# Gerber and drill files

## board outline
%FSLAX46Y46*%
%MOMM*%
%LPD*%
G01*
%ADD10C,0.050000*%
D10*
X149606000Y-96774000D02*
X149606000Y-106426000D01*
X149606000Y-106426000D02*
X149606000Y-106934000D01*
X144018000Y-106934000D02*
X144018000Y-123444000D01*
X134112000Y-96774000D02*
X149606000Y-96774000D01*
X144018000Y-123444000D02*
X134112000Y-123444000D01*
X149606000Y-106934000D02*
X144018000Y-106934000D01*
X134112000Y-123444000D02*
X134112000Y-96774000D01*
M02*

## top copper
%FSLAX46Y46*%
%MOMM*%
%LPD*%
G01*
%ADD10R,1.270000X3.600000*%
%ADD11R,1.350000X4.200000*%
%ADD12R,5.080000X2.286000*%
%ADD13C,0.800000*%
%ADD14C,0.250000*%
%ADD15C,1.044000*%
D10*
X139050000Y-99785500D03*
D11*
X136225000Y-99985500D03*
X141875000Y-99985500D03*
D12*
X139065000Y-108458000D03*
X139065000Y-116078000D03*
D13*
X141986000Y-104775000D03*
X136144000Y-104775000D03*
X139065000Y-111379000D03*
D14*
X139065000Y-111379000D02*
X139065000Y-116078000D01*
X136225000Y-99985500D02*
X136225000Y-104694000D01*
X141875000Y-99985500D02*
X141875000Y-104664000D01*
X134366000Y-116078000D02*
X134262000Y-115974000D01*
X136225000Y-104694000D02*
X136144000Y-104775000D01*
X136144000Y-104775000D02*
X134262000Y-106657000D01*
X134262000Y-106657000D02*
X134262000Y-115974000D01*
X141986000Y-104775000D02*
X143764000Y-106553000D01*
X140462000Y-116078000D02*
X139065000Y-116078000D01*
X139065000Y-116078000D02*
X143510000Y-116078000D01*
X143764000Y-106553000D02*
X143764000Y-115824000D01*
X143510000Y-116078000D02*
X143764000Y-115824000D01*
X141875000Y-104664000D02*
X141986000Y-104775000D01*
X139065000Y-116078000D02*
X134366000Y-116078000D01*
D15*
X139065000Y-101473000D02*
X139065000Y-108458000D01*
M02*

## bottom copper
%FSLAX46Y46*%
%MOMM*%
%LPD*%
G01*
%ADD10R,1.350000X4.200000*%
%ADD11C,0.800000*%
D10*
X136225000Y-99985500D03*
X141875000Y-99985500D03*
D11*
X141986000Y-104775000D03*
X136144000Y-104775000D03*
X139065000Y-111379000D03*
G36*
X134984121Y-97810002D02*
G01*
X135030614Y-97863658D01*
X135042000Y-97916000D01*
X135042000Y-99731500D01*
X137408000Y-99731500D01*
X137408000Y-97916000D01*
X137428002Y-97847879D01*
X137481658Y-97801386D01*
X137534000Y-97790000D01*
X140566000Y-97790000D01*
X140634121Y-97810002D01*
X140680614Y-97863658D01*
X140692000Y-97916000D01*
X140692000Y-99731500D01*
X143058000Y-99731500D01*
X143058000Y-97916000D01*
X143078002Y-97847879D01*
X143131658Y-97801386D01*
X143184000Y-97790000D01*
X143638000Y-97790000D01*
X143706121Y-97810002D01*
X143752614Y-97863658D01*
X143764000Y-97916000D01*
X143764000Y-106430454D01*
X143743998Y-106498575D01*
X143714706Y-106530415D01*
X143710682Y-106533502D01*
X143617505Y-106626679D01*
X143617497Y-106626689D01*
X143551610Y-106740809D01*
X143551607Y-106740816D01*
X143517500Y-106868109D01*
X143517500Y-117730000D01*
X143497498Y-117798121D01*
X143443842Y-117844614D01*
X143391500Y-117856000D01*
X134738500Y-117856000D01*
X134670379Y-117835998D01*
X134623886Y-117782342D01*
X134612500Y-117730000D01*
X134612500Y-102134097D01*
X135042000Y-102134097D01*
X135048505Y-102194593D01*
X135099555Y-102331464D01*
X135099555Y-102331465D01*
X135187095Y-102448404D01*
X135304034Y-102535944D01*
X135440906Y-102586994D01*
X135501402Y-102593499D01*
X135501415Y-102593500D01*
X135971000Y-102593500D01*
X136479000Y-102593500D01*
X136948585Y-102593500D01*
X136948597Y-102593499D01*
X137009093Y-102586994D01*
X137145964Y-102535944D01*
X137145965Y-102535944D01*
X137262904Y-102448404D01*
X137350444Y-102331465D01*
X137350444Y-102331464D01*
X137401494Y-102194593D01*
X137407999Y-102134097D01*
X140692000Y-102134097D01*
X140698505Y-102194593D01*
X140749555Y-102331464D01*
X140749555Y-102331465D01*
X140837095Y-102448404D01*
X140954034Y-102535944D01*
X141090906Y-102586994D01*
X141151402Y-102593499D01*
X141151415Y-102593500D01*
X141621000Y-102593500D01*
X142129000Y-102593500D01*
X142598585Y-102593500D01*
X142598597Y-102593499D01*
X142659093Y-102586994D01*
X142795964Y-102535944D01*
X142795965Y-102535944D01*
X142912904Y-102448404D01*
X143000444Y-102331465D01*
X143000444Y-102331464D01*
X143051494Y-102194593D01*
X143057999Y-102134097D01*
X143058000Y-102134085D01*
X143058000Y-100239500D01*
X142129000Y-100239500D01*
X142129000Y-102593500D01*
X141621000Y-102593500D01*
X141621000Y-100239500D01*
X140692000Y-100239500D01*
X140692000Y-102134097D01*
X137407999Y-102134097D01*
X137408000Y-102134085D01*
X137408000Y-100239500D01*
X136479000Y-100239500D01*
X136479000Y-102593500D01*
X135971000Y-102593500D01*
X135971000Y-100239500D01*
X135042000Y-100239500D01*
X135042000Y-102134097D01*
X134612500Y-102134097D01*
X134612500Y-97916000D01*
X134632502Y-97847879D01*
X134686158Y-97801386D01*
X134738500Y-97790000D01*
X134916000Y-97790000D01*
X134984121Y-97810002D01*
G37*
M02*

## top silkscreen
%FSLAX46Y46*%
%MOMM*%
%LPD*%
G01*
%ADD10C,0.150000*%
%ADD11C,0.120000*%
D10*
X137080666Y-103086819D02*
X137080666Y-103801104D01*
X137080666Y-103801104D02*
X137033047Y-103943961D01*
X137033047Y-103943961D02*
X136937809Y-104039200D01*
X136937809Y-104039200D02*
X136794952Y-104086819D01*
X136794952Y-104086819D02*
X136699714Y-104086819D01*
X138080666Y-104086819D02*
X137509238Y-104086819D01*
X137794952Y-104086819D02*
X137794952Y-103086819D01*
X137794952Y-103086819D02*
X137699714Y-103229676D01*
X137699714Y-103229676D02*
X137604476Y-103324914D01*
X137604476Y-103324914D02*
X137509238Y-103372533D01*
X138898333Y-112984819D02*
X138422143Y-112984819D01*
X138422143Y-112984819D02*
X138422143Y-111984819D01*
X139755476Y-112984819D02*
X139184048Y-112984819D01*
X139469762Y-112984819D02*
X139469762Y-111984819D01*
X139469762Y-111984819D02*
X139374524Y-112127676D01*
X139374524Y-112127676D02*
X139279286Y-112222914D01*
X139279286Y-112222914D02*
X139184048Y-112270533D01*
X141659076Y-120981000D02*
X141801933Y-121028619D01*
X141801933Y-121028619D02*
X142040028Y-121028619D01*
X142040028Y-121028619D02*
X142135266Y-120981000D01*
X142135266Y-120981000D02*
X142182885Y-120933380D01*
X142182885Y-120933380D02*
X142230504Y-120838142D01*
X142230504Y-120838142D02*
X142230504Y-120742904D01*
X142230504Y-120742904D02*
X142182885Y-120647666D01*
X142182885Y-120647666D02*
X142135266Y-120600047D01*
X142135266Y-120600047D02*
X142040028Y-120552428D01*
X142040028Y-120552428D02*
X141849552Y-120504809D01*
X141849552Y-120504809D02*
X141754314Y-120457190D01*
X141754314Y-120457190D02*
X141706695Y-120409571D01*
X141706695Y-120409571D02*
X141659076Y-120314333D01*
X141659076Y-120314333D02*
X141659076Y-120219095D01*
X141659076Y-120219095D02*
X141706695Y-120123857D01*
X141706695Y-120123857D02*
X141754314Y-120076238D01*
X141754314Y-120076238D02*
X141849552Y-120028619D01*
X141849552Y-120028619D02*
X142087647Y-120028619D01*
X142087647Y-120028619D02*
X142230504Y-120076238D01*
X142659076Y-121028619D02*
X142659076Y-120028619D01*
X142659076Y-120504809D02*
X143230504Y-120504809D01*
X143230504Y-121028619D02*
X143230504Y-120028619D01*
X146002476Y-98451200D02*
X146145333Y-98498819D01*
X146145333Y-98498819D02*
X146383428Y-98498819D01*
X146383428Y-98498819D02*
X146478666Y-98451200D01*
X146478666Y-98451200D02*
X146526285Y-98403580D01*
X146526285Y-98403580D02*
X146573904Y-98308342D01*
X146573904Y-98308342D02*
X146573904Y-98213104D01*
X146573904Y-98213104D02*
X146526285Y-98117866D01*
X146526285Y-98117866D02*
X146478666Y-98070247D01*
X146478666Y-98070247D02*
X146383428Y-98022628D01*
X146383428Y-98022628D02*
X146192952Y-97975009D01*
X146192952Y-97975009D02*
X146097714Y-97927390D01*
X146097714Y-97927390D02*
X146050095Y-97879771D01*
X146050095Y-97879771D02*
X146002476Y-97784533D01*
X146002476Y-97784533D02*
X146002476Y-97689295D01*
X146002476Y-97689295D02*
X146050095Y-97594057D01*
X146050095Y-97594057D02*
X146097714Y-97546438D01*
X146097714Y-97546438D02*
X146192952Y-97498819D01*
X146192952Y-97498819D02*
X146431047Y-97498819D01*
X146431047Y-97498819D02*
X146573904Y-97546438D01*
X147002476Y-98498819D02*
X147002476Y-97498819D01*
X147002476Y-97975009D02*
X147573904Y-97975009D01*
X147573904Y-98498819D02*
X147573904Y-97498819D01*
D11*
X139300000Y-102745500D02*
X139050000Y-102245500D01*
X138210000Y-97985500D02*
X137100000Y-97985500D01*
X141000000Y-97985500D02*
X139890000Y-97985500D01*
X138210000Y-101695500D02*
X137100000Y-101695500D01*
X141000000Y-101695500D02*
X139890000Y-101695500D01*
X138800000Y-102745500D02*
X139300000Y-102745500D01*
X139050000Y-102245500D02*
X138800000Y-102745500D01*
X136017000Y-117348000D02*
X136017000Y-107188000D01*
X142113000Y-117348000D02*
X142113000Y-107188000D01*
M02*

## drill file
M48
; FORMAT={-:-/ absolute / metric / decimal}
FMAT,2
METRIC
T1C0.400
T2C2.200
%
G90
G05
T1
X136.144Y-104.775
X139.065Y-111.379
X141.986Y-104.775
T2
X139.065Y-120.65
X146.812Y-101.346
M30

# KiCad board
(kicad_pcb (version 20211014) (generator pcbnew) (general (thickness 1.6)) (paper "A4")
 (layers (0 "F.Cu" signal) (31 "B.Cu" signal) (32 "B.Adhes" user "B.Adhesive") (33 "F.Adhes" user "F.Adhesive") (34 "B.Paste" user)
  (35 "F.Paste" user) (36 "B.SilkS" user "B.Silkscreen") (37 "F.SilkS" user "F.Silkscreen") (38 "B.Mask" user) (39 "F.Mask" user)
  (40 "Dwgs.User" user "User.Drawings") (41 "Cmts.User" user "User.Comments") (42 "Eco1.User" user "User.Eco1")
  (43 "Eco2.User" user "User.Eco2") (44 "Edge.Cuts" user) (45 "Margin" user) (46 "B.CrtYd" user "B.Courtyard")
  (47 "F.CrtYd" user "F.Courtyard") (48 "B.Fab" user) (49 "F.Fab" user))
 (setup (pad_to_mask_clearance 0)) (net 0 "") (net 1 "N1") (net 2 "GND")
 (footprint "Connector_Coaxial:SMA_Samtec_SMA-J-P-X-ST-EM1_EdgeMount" (layer "F.Cu") (at 139.05 99.9855 180)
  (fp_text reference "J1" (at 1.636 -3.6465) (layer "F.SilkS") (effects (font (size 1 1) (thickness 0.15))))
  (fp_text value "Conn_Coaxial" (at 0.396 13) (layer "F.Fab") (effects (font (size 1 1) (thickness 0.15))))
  (fp_line (start -0.25 -2.76) (end 0 -2.26) (layer "F.SilkS") (width 0.12))
  (fp_line (start 0.84 2) (end 1.95 2) (layer "F.SilkS") (width 0.12))
  (fp_line (start -1.95 2) (end -0.84 2) (layer "F.SilkS") (width 0.12))
  (fp_line (start 0.84 -1.71) (end 1.95 -1.71) (layer "F.SilkS") (width 0.12))
  (fp_line (start -1.95 -1.71) (end -0.84 -1.71) (layer "F.SilkS") (width 0.12))
  (fp_line (start 0.25 -2.76) (end -0.25 -2.76) (layer "F.SilkS") (width 0.12))
  (fp_line (start 0 -2.26) (end 0.25 -2.76) (layer "F.SilkS") (width 0.12))
  (pad "1" smd rect (at 0 0.2 180) (size 1.27 3.6) (layers "F.Cu" "F.Paste" "F.Mask") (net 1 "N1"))
  (pad "2" smd rect (at 2.825 0 180) (size 1.35 4.2) (layers "B.Cu" "B.Paste" "B.Mask") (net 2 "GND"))
  (pad "2" smd rect (at 2.825 0 180) (size 1.35 4.2) (layers "F.Cu" "F.Paste" "F.Mask") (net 2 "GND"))
  (pad "2" smd rect (at -2.825 0 180) (size 1.35 4.2) (layers "B.Cu" "B.Paste" "B.Mask") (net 2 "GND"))
  (pad "2" smd rect (at -2.825 0 180) (size 1.35 4.2) (layers "F.Cu" "F.Paste" "F.Mask") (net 2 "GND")))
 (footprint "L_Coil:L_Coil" (layer "F.Cu") (at 139.065 109.474 180)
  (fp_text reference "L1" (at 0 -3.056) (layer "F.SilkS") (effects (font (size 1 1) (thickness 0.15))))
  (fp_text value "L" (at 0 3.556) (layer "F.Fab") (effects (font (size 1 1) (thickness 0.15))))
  (fp_line (start 3.048 -7.874) (end 3.048 2.286) (layer "F.SilkS") (width 0.12))
  (fp_line (start -3.048 -7.874) (end -3.048 2.286) (layer "F.SilkS") (width 0.12))
  (pad "1" smd rect locked (at 0 1.016 180) (size 5.08 2.286) (layers "F.Cu" "F.Paste" "F.Mask") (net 1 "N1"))
  (pad "2" smd rect locked (at 0 -6.604 180) (size 5.08 2.286) (layers "F.Cu" "F.Paste" "F.Mask") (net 2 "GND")))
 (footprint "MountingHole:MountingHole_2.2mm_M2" (layer "F.Cu") (at 139.065 120.65)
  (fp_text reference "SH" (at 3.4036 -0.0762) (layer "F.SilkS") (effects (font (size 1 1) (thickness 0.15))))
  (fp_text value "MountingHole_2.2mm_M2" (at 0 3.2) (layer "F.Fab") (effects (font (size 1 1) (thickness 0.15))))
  (pad "" np_thru_hole circle (at 0 0) (size 2.2 2.2) (drill 2.2) (layers *.Cu *.Mask)))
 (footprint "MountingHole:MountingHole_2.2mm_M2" (layer "F.Cu") (at 146.812 101.346)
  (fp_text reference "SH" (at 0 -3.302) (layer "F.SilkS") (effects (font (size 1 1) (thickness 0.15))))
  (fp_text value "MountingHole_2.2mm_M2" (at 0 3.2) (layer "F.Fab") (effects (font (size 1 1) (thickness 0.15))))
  (pad "" np_thru_hole circle (at 0 0) (size 2.2 2.2) (drill 2.2) (layers *.Cu *.Mask)))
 (gr_line (start 149.606 96.774) (end 149.606 106.426) (layer "Edge.Cuts") (width 0.05))
 (gr_line (start 149.606 106.426) (end 149.606 106.934) (layer "Edge.Cuts") (width 0.05))
 (gr_line (start 144.018 106.934) (end 144.018 123.444) (layer "Edge.Cuts") (width 0.05))
 (gr_line (start 134.112 96.774) (end 149.606 96.774) (layer "Edge.Cuts") (width 0.05))
 (gr_line (start 144.018 123.444) (end 134.112 123.444) (layer "Edge.Cuts") (width 0.05))
 (gr_line (start 149.606 106.934) (end 144.018 106.934) (layer "Edge.Cuts") (width 0.05))
 (gr_line (start 134.112 123.444) (end 134.112 96.774) (layer "Edge.Cuts") (width 0.05))
 (segment (start 139.065 111.379) (end 139.065 116.078) (width 0.25) (layer "F.Cu") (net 2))
 (segment (start 136.225 99.9855) (end 136.225 104.694) (width 0.25) (layer "F.Cu") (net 2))
 (segment (start 141.875 99.9855) (end 141.875 104.664) (width 0.25) (layer "F.Cu") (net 2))
 (segment (start 134.366 116.078) (end 134.262 115.974) (width 0.25) (layer "F.Cu") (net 2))
 (segment (start 136.225 104.694) (end 136.144 104.775) (width 0.25) (layer "F.Cu") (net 2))
 (segment (start 136.144 104.775) (end 134.262 106.657) (width 0.25) (layer "F.Cu") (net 2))
 (segment (start 134.262 106.657) (end 134.262 115.974) (width 0.25) (layer "F.Cu") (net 2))
 (segment (start 141.986 104.775) (end 143.764 106.553) (width 0.25) (layer "F.Cu") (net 2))
 (segment (start 140.462 116.078) (end 139.065 116.078) (width 0.25) (layer "F.Cu") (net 2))
 (segment (start 139.065 116.078) (end 143.51 116.078) (width 0.25) (layer "F.Cu") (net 2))
 (segment (start 143.764 106.553) (end 143.764 115.824) (width 0.25) (layer "F.Cu") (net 2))
 (segment (start 143.51 116.078) (end 143.764 115.824) (width 0.25) (layer "F.Cu") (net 2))
 (segment (start 141.875 104.664) (end 141.986 104.775) (width 0.25) (layer "F.Cu") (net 2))
 (segment (start 139.065 116.078) (end 134.366 116.078) (width 0.25) (layer "F.Cu") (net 2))
 (via (at 141.986 104.775) (size 0.8) (drill 0.4) (layers "F.Cu" "B.Cu") (free) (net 2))
 (via (at 136.144 104.775) (size 0.8) (drill 0.4) (layers "F.Cu" "B.Cu") (free) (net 2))
 (via (at 139.065 111.379) (size 0.8) (drill 0.4) (layers "F.Cu" "B.Cu") (free) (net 2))
 (segment (start 139.065 101.473) (end 139.065 108.458) (width 1.044) (layer "F.Cu") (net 1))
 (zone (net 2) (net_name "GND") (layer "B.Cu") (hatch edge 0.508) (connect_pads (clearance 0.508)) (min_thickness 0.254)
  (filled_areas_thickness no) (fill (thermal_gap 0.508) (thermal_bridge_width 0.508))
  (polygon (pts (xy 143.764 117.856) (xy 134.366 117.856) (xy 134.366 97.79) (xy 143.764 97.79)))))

